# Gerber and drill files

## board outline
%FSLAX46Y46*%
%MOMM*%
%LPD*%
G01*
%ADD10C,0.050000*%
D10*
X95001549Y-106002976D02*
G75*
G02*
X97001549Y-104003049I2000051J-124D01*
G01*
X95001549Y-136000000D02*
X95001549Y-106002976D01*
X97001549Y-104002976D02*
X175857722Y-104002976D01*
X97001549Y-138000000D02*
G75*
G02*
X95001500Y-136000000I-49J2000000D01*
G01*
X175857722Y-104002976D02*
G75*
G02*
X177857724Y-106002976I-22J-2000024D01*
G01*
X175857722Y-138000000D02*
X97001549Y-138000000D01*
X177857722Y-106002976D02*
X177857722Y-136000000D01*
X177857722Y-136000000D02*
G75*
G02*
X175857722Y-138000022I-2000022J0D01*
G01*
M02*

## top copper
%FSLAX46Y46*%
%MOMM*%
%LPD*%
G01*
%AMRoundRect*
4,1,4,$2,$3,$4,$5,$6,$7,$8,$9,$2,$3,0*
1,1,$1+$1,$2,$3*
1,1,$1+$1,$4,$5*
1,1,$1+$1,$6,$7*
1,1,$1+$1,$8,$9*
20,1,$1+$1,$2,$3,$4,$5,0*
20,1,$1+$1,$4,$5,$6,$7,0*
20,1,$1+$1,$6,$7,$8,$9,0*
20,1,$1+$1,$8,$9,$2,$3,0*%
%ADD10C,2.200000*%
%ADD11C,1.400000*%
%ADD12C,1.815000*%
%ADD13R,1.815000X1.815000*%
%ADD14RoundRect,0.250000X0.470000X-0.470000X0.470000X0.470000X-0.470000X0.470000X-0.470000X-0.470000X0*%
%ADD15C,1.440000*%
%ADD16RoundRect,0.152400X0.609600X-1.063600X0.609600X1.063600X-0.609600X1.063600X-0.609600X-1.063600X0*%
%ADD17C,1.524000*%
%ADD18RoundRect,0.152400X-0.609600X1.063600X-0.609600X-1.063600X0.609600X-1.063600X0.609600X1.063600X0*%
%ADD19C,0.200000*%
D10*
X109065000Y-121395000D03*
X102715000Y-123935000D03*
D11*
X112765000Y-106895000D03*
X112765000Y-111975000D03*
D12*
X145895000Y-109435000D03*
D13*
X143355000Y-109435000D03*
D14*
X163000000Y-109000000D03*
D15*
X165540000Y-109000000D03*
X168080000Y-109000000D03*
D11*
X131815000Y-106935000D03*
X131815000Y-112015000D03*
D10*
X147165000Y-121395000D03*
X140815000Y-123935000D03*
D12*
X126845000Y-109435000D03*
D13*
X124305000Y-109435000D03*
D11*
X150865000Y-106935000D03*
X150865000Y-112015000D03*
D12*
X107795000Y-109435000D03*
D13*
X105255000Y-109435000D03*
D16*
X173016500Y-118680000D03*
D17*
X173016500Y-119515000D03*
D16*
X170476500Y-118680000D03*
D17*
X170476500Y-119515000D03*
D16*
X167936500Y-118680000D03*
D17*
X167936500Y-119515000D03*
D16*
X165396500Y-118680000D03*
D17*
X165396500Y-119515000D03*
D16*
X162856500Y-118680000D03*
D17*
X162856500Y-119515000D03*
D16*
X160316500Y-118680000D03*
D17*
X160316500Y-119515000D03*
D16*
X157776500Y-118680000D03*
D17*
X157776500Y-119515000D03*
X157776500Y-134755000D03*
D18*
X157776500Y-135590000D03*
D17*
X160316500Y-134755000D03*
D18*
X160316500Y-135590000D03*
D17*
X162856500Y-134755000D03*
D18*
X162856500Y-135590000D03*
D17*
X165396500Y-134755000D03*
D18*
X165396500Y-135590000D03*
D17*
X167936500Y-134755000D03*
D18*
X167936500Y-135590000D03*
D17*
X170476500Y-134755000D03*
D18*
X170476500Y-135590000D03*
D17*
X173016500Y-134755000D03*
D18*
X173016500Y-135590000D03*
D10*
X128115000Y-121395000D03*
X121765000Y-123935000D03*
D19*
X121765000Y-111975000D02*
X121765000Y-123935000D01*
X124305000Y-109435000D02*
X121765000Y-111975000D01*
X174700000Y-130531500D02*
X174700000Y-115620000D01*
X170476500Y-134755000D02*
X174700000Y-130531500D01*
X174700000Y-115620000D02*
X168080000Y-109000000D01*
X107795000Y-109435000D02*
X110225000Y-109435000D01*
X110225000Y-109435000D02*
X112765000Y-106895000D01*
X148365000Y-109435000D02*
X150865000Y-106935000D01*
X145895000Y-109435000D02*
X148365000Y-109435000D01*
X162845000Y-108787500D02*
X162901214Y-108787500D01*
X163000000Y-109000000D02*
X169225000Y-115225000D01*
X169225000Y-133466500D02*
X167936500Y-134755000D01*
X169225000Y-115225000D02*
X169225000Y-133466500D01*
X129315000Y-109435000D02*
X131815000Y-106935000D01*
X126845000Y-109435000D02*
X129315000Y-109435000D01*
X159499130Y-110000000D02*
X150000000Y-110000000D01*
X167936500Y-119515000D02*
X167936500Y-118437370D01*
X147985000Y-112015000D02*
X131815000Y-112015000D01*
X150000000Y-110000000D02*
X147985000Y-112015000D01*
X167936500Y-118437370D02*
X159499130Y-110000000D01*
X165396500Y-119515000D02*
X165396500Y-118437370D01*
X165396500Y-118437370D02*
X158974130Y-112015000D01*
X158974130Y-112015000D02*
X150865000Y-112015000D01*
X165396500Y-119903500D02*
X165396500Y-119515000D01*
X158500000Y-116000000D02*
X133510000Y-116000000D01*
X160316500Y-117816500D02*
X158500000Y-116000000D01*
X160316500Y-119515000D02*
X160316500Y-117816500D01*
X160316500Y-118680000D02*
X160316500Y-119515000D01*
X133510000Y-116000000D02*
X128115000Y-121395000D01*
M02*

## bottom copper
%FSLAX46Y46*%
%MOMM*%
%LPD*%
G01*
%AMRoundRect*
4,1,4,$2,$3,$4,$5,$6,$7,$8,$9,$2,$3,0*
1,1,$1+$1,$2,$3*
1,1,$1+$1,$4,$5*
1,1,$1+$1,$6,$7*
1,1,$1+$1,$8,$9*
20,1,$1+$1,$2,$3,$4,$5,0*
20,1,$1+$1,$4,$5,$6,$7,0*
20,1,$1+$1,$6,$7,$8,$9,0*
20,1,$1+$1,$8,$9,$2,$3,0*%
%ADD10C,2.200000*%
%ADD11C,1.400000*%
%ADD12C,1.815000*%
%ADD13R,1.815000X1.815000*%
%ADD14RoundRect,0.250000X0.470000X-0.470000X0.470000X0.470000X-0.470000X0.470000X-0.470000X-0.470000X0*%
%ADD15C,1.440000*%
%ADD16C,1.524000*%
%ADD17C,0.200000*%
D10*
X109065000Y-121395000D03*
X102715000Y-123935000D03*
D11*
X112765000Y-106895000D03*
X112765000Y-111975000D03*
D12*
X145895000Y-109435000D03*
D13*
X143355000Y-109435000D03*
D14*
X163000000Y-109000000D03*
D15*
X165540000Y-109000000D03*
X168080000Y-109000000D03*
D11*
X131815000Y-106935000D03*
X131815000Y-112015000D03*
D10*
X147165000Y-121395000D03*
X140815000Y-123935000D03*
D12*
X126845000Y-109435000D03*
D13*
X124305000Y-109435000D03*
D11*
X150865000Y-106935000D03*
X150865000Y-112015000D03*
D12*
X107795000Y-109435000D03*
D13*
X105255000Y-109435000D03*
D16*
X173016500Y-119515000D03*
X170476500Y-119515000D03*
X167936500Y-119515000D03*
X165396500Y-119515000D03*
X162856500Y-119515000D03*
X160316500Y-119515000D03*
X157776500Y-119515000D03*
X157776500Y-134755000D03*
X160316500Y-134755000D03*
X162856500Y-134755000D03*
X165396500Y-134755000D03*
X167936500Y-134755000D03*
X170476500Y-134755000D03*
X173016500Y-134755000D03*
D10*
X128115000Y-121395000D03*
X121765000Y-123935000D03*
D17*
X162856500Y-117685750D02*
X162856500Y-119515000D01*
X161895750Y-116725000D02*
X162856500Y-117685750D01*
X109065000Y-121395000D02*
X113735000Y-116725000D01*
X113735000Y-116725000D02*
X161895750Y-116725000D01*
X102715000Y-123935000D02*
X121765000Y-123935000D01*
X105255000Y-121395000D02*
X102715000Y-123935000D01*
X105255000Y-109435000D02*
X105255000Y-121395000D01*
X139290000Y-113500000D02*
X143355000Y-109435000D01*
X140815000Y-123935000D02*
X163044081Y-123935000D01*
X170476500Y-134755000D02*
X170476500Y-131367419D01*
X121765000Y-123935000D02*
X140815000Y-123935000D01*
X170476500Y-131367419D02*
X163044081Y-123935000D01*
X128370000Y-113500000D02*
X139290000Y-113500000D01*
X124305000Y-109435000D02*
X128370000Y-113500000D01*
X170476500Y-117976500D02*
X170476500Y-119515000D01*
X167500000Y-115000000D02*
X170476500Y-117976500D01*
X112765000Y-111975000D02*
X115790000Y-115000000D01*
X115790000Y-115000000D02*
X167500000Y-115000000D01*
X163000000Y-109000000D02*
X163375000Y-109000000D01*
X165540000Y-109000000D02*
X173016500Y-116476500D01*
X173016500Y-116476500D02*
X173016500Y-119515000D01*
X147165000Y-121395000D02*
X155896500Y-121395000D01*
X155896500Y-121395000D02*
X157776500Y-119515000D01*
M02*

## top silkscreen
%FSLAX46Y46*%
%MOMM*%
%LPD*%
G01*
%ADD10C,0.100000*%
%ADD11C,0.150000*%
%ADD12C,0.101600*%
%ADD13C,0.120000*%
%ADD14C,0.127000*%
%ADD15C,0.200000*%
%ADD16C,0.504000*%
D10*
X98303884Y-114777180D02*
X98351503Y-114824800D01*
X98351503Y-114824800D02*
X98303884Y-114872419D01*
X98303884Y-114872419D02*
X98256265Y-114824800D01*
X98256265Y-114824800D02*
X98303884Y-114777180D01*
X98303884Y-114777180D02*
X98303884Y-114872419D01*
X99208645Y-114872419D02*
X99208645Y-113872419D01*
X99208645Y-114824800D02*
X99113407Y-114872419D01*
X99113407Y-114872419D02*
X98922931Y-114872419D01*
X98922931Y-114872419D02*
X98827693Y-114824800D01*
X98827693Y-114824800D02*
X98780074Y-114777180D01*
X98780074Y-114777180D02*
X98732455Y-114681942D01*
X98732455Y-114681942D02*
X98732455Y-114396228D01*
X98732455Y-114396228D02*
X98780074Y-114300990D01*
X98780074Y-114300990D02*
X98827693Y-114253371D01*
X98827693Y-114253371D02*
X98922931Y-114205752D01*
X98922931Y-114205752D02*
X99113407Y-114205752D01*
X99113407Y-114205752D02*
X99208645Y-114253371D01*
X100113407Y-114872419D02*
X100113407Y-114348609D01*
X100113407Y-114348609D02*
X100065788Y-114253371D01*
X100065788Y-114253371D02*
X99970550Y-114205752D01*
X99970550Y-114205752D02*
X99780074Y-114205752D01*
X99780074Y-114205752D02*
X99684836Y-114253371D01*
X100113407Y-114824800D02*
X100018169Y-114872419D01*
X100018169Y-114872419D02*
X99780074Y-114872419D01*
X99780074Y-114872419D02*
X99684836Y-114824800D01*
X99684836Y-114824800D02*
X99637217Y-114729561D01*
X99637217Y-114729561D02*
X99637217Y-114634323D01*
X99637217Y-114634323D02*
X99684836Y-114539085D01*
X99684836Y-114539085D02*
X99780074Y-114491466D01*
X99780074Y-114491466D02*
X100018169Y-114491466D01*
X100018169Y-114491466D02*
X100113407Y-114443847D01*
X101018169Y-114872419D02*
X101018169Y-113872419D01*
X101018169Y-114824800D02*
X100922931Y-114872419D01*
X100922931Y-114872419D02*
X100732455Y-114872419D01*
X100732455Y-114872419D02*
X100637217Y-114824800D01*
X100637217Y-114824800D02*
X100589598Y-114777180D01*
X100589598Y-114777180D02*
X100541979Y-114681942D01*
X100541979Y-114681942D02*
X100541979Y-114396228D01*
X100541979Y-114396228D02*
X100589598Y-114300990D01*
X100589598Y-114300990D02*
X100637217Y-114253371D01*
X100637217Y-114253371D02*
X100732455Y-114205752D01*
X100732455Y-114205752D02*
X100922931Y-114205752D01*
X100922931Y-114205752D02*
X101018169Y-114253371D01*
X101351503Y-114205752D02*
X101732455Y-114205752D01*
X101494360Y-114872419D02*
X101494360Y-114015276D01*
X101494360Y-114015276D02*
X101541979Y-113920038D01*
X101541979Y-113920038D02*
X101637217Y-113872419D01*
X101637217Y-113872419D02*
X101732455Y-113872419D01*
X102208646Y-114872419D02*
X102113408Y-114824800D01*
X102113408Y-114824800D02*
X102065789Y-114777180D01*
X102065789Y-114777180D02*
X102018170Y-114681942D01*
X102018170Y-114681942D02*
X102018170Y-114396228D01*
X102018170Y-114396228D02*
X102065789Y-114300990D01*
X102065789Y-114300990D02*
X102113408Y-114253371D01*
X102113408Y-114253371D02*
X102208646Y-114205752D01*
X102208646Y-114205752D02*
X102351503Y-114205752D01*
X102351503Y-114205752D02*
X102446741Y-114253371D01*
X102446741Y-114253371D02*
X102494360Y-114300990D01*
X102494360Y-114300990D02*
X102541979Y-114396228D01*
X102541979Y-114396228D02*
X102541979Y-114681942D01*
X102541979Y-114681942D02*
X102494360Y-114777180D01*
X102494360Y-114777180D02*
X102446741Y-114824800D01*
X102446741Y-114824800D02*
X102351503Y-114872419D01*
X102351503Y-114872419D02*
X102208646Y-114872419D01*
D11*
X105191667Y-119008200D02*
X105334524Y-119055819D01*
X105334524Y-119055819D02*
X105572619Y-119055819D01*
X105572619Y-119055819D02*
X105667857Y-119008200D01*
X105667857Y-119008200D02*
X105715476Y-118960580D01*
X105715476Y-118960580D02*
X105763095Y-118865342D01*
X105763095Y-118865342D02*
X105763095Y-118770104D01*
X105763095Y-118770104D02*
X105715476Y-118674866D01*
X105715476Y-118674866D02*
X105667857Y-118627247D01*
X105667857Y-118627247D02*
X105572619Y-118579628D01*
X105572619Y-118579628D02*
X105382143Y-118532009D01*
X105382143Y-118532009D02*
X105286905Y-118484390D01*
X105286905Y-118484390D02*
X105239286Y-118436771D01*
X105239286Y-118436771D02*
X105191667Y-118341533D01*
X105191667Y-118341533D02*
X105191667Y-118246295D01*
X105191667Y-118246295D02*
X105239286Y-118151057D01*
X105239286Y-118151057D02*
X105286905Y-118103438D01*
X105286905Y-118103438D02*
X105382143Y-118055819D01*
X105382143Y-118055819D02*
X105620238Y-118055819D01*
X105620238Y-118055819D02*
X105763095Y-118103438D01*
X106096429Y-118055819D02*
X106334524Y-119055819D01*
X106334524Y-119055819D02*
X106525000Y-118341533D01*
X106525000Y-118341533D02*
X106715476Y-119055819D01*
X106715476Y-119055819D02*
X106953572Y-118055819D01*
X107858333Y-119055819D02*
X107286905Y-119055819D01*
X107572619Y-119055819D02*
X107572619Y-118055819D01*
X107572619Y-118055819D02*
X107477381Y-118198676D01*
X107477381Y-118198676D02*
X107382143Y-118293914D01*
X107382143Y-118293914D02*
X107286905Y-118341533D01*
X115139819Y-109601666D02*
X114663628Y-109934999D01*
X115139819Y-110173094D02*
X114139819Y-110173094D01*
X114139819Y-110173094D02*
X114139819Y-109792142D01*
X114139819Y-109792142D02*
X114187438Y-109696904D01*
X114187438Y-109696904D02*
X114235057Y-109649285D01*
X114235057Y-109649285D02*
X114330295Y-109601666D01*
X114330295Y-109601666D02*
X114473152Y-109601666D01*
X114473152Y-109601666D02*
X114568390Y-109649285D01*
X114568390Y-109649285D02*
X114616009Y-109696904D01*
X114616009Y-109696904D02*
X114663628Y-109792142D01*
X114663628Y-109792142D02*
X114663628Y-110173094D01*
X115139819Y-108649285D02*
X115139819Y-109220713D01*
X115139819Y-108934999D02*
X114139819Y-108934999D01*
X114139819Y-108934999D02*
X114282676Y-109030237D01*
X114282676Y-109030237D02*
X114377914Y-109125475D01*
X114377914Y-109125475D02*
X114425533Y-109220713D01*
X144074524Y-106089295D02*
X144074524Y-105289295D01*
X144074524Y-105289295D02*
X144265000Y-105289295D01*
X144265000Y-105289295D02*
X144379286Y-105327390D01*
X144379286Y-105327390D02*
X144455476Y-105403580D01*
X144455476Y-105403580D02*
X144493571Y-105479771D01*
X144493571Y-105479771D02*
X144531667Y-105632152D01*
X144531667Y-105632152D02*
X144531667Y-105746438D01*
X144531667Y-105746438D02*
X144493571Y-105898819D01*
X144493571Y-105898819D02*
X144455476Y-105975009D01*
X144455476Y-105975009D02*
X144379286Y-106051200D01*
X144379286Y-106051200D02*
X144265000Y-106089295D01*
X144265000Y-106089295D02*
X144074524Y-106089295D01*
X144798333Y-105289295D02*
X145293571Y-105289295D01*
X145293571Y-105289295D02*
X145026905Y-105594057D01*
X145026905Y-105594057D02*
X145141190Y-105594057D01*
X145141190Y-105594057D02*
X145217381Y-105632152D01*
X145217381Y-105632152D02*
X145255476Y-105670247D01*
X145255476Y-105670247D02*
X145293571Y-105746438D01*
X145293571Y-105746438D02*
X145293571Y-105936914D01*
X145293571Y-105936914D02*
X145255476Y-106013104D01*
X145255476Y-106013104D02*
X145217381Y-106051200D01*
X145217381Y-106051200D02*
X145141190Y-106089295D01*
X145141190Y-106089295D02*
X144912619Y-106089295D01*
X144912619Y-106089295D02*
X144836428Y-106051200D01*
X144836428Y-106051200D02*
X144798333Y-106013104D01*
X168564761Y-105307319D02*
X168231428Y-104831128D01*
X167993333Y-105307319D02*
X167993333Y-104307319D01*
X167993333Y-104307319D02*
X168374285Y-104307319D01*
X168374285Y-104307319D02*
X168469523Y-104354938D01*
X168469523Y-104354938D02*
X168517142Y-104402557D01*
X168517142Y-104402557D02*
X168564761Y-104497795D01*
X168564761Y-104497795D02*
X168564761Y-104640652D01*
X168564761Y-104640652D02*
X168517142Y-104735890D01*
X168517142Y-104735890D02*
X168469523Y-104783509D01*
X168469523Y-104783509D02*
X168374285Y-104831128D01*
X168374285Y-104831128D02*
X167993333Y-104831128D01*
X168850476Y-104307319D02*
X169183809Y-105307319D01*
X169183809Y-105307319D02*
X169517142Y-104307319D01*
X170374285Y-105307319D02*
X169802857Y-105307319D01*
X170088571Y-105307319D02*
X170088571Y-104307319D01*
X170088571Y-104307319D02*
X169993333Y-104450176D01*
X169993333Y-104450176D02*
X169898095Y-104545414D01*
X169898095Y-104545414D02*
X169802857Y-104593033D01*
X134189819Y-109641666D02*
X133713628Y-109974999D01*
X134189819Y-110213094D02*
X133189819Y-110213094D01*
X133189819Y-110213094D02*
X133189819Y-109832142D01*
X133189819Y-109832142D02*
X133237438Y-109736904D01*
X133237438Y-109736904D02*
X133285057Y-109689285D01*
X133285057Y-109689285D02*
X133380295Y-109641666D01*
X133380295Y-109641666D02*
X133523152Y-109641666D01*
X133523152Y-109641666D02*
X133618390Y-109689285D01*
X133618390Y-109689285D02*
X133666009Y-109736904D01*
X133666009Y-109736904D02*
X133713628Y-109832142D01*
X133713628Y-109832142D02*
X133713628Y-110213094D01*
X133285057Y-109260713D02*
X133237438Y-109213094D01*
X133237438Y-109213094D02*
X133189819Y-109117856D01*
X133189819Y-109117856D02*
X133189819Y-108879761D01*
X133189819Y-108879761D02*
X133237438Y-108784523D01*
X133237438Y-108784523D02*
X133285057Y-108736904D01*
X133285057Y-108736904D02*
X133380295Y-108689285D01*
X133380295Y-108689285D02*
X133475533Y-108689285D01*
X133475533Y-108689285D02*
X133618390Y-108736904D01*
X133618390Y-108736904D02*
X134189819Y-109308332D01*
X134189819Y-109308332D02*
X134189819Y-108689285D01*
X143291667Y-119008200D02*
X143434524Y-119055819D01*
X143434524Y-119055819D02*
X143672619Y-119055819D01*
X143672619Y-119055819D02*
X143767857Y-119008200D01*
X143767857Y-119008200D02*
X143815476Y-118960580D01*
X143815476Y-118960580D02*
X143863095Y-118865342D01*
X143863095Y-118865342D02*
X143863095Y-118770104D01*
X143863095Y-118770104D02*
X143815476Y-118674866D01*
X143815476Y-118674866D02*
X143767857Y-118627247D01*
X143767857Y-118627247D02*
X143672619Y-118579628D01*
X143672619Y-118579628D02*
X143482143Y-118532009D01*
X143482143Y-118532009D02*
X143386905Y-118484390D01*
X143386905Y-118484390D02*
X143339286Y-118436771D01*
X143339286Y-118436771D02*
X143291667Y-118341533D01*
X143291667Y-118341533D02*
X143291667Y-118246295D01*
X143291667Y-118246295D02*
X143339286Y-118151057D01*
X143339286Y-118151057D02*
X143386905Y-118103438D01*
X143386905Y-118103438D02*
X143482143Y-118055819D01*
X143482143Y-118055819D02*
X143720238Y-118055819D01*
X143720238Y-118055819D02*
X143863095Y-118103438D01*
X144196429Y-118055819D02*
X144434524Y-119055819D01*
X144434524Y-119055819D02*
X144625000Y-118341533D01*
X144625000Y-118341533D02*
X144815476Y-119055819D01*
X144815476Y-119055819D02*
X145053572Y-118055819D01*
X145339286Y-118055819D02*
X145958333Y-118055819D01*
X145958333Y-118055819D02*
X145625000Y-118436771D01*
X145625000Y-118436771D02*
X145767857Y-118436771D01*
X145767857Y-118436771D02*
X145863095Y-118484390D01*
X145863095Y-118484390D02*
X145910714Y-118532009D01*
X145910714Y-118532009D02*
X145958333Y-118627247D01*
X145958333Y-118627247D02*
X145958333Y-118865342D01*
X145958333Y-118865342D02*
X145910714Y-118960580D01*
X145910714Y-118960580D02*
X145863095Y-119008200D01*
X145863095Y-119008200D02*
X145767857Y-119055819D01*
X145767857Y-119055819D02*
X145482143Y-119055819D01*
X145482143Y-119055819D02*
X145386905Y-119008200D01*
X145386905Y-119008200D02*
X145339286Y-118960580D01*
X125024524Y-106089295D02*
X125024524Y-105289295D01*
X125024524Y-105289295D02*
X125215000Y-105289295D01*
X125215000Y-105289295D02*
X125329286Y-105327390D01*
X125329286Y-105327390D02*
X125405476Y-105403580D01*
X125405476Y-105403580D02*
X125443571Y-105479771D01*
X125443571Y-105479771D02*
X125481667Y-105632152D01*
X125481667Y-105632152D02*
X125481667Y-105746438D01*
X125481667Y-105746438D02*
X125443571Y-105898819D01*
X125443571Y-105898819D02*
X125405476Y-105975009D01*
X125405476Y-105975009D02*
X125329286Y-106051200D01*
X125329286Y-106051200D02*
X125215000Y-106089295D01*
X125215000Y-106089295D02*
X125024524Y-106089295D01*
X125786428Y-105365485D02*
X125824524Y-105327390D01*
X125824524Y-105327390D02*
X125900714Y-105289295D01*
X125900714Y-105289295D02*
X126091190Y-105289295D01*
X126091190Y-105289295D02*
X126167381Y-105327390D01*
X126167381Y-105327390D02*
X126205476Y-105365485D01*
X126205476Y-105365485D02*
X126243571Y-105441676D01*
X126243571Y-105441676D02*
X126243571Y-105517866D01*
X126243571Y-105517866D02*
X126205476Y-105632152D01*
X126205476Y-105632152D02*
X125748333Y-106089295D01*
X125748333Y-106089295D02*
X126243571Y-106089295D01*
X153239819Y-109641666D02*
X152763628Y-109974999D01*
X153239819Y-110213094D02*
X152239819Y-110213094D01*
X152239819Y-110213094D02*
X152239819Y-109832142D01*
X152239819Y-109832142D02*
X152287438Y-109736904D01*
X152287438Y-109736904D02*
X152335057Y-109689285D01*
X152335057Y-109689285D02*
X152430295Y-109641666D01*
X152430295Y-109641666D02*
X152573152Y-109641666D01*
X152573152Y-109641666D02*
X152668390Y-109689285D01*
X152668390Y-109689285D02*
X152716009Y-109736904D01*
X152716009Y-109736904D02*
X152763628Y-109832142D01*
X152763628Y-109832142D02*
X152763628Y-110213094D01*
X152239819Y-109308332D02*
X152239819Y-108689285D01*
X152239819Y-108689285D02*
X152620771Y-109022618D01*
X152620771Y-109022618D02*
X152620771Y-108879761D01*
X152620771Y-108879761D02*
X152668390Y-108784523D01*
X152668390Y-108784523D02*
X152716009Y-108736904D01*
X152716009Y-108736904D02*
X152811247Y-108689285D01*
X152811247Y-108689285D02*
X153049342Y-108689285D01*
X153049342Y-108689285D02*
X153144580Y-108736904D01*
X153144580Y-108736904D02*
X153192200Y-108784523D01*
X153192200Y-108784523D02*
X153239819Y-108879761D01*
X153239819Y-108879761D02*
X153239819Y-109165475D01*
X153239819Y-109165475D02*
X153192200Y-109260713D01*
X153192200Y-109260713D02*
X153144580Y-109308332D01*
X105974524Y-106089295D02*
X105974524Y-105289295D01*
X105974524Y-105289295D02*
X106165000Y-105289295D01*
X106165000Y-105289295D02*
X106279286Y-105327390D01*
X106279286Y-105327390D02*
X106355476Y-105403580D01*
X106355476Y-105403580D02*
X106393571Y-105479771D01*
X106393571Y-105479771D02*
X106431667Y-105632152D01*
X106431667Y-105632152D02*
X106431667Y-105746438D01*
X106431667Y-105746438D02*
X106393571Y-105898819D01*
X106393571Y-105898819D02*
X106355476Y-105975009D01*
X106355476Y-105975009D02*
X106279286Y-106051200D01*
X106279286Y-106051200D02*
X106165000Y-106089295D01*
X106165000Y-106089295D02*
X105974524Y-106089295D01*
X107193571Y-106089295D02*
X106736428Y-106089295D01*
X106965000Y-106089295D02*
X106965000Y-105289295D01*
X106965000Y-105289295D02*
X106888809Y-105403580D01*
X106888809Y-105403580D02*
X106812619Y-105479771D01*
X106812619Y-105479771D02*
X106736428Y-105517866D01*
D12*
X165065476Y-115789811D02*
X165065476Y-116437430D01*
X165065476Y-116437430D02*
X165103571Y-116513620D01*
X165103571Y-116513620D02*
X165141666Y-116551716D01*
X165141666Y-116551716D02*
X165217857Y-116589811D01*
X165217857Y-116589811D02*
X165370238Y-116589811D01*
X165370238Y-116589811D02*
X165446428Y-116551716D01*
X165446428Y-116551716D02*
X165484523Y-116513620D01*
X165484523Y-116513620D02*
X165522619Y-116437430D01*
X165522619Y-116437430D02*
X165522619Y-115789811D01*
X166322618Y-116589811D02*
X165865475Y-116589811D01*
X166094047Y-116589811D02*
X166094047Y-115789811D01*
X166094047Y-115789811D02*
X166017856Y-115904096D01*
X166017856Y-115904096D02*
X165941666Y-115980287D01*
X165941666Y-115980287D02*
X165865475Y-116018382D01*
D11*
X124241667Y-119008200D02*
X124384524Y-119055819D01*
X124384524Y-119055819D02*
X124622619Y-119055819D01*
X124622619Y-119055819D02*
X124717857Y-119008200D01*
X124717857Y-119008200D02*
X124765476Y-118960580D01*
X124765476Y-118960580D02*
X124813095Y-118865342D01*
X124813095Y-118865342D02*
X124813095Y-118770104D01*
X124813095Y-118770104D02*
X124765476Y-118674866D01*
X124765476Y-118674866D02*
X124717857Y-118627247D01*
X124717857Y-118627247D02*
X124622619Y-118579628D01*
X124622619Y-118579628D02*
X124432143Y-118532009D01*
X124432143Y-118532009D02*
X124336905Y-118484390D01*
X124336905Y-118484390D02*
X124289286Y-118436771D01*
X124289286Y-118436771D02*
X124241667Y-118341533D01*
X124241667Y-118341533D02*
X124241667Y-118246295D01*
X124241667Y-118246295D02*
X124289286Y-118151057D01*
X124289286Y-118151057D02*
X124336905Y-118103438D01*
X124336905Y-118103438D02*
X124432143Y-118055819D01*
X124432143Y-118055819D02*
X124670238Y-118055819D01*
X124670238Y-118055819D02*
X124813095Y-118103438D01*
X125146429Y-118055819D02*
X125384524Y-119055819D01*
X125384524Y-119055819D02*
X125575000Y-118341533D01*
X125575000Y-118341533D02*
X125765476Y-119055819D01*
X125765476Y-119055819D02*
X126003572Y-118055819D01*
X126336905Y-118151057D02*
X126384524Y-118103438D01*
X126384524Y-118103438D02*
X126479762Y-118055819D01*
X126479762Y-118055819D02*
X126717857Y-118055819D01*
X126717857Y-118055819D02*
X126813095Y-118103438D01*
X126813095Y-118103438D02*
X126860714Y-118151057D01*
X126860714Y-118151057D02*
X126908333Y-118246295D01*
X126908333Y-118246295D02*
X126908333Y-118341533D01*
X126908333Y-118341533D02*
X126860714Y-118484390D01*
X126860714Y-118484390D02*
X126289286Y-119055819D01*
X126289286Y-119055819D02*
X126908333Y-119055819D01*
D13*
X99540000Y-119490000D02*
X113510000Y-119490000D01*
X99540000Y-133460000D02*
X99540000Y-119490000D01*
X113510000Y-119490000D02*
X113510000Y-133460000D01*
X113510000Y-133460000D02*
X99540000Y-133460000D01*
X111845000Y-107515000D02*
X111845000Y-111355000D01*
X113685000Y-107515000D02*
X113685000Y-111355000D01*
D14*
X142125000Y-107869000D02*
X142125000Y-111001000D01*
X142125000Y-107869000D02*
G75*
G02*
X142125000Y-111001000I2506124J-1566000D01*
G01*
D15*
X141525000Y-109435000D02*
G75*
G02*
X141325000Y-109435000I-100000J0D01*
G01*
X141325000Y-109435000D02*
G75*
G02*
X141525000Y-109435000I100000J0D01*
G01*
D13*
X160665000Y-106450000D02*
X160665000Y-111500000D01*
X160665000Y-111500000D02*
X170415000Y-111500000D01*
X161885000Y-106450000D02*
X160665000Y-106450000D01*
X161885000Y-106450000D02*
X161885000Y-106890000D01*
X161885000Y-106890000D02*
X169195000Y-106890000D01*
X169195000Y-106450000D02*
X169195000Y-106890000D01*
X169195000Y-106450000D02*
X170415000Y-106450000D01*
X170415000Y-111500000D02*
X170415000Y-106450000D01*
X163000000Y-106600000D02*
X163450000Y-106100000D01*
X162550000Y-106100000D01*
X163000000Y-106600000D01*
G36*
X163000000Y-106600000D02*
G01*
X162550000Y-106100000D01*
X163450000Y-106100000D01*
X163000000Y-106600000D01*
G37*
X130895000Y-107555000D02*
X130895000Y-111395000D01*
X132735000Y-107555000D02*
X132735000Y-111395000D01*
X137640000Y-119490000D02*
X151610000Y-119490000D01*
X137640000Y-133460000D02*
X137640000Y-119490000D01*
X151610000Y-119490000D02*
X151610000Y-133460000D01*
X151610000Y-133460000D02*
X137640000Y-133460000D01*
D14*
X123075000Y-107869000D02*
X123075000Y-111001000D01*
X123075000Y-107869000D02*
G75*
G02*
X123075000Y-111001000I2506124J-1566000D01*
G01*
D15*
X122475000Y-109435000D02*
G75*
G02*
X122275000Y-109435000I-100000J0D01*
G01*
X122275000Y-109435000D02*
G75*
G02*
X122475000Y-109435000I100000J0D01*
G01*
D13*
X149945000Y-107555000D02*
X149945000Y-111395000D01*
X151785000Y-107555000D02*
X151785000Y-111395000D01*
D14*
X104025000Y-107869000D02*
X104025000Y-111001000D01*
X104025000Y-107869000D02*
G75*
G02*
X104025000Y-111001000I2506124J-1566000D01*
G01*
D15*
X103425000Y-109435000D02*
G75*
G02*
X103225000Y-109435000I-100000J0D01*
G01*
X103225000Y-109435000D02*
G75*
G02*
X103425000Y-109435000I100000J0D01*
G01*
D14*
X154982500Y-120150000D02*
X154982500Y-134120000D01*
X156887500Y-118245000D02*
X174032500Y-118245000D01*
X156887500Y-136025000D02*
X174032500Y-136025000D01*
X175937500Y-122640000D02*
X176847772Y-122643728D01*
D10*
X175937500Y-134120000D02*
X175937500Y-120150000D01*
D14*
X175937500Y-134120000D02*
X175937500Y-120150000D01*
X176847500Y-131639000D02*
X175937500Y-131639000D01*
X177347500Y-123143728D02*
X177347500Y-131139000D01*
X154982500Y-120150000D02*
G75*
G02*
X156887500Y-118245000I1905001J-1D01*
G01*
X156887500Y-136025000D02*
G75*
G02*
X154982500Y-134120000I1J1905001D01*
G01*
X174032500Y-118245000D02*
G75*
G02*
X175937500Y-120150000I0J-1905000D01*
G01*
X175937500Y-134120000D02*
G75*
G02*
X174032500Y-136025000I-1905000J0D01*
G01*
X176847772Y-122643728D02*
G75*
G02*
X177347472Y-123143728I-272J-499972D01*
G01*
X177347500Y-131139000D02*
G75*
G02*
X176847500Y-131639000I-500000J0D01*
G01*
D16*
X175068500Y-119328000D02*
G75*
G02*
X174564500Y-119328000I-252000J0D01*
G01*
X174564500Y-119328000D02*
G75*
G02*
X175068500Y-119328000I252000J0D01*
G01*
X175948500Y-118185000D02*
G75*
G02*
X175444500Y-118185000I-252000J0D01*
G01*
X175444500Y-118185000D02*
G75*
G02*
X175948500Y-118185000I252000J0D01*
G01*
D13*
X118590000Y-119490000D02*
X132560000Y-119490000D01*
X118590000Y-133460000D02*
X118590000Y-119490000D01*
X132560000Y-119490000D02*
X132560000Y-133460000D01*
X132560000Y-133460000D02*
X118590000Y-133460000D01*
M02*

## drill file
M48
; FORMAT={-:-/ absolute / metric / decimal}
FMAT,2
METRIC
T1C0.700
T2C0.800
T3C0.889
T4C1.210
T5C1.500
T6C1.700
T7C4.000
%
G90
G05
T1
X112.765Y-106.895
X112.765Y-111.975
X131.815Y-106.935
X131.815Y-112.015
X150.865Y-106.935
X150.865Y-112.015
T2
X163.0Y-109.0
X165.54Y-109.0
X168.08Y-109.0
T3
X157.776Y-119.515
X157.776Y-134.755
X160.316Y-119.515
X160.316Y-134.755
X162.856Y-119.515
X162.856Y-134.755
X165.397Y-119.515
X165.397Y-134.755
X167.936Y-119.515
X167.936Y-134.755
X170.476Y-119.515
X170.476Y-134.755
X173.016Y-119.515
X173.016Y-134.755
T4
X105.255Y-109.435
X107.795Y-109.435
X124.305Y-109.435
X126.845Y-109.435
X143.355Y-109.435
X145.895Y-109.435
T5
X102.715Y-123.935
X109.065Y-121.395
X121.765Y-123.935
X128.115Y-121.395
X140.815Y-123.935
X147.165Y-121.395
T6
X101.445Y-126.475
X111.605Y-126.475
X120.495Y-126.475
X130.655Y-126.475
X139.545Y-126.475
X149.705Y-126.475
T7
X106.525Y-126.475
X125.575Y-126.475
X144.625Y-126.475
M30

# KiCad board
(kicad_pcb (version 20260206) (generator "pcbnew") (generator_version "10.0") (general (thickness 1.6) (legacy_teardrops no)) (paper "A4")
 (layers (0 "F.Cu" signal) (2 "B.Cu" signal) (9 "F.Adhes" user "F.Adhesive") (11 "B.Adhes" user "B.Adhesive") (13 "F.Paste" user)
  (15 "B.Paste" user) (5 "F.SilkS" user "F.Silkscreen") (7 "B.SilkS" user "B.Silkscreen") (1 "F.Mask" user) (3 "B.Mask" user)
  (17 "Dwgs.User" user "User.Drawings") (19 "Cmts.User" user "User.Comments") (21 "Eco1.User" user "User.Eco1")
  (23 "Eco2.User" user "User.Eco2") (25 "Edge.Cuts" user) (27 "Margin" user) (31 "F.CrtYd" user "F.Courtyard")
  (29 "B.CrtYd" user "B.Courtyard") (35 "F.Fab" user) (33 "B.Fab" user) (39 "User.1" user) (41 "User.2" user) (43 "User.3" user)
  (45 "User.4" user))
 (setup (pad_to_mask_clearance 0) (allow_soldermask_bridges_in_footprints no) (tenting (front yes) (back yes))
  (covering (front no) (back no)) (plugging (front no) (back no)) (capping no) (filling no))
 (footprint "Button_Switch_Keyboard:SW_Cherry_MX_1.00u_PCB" (layer "F.Cu") (at 109.065 121.395)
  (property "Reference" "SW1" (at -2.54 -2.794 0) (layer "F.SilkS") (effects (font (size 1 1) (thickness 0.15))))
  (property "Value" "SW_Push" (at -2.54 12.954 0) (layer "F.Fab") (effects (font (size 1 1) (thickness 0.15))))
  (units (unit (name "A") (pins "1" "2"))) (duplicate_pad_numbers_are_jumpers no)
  (fp_line (start -9.525 -1.905) (end 4.445 -1.905) (stroke (width 0.12) (type solid)) (layer "F.SilkS"))
  (fp_line (start -9.525 12.065) (end -9.525 -1.905) (stroke (width 0.12) (type solid)) (layer "F.SilkS"))
  (fp_line (start 4.445 -1.905) (end 4.445 12.065) (stroke (width 0.12) (type solid)) (layer "F.SilkS"))
  (fp_line (start 4.445 12.065) (end -9.525 12.065) (stroke (width 0.12) (type solid)) (layer "F.SilkS"))
  (pad "" np_thru_hole circle (at -7.62 5.08) (size 1.7 1.7) (drill 1.7) (layers "*.Cu" "*.Mask"))
  (pad "" np_thru_hole circle (at -2.54 5.08) (size 4 4) (drill 4) (layers "*.Cu" "*.Mask"))
  (pad "" np_thru_hole circle (at 2.54 5.08) (size 1.7 1.7) (drill 1.7) (layers "*.Cu" "*.Mask"))
  (pad "1" thru_hole circle (at 0 0) (size 2.2 2.2) (drill 1.5) (layers "*.Cu" "*.Mask") (remove_unused_layers no) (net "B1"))
  (pad "2" thru_hole circle (at -6.35 2.54) (size 2.2 2.2) (drill 1.5) (layers "*.Cu" "*.Mask") (remove_unused_layers no) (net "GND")))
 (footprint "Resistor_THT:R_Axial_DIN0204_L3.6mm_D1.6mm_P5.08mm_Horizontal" (layer "F.Cu") (at 112.765 106.895 -90)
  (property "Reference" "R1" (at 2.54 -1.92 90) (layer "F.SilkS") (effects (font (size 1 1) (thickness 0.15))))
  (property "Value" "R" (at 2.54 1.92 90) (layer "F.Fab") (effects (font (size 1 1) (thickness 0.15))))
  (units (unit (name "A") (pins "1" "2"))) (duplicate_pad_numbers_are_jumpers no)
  (fp_line (start 0.62 0.92) (end 4.46 0.92) (stroke (width 0.12) (type solid)) (layer "F.SilkS"))
  (fp_line (start 0.62 -0.92) (end 4.46 -0.92) (stroke (width 0.12) (type solid)) (layer "F.SilkS"))
  (pad "1" thru_hole circle (at 0 0 270) (size 1.4 1.4) (drill 0.7) (layers "*.Cu" "*.Mask") (remove_unused_layers no) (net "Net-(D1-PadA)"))
  (pad "2" thru_hole circle (at 5.08 0 270) (size 1.4 1.4) (drill 0.7) (layers "*.Cu" "*.Mask") (remove_unused_layers no) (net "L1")))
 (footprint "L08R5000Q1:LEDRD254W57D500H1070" (layer "F.Cu") (at 144.625 109.435)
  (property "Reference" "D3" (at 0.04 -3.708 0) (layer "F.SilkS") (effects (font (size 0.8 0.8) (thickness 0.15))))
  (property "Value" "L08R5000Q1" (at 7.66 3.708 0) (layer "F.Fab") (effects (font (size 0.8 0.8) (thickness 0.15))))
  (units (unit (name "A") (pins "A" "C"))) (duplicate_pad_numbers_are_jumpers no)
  (fp_line (start -2.5 -1.566) (end -2.5 1.566) (stroke (width 0.127) (type solid)) (layer "F.SilkS"))
  (fp_arc (start -2.5 -1.566) (mid 2.961291 0) (end -2.5 1.566) (stroke (width 0.127) (type solid)) (layer "F.SilkS"))
  (fp_circle (center -3.2 0) (end -3.1 0) (stroke (width 0.2) (type solid)) (fill no) (layer "F.SilkS"))
  (pad "A" thru_hole circle (at 1.27 0) (size 1.815 1.815) (drill 1.21) (layers "*.Cu" "*.Mask") (remove_unused_layers no)
   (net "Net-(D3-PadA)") (solder_mask_margin 0.102))
  (pad "C" thru_hole rect (at -1.27 0) (size 1.815 1.815) (drill 1.21) (layers "*.Cu" "*.Mask") (remove_unused_layers no) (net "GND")
   (solder_mask_margin 0.102)))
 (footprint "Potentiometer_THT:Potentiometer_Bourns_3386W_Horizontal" (layer "F.Cu") (at 163 109)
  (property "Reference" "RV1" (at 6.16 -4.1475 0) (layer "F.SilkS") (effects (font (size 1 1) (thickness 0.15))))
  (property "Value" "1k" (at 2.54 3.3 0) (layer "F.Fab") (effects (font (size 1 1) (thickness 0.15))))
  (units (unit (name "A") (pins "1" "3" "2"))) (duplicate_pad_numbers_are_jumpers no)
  (fp_line (start -2.335 -2.55) (end -2.335 2.5) (stroke (width 0.12) (type default)) (layer "F.SilkS"))
  (fp_line (start -2.335 2.5) (end 7.415 2.5) (stroke (width 0.12) (type default)) (layer "F.SilkS"))
  (fp_line (start -1.115 -2.55) (end -2.335 -2.55) (stroke (width 0.12) (type default)) (layer "F.SilkS"))
  (fp_line (start -1.115 -2.55) (end -1.115 -2.11) (stroke (width 0.12) (type default)) (layer "F.SilkS"))
  (fp_line (start -1.115 -2.11) (end 6.195 -2.11) (stroke (width 0.12) (type default)) (layer "F.SilkS"))
  (fp_line (start 6.195 -2.55) (end 6.195 -2.11) (stroke (width 0.12) (type default)) (layer "F.SilkS"))
  (fp_line (start 6.195 -2.55) (end 7.415 -2.55) (stroke (width 0.12) (type default)) (layer "F.SilkS"))
  (fp_line (start 7.415 2.5) (end 7.415 -2.55) (stroke (width 0.12) (type default)) (layer "F.SilkS"))
  (fp_poly (pts (xy 0 -2.4) (xy 0.45 -2.9) (xy -0.45 -2.9)) (stroke (width 0.12) (type solid)) (fill yes) (layer "F.SilkS"))
  (pad "1" thru_hole roundrect (at 0 0 90) (size 1.44 1.44) (drill 0.8) (layers "*.Cu" "*.Mask") (remove_unused_layers no)
   (roundrect_rratio 0.1736111111) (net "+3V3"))
  (pad "2" thru_hole circle (at 2.54 0 90) (size 1.44 1.44) (drill 0.8) (layers "*.Cu" "*.Mask") (remove_unused_layers no) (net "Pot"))
  (pad "3" thru_hole circle (at 5.08 0 90) (size 1.44 1.44) (drill 0.8) (layers "*.Cu" "*.Mask") (remove_unused_layers no) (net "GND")))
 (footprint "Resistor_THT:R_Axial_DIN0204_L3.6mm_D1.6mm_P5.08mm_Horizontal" (layer "F.Cu") (at 131.815 106.935 -90)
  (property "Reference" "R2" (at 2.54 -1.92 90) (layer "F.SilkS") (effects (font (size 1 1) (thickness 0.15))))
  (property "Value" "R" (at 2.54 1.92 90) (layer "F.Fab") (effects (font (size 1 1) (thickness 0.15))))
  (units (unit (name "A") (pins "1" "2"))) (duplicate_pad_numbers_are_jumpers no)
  (fp_line (start 0.62 0.92) (end 4.46 0.92) (stroke (width 0.12) (type solid)) (layer "F.SilkS"))
  (fp_line (start 0.62 -0.92) (end 4.46 -0.92) (stroke (width 0.12) (type solid)) (layer "F.SilkS"))
  (pad "1" thru_hole circle (at 0 0 270) (size 1.4 1.4) (drill 0.7) (layers "*.Cu" "*.Mask") (remove_unused_layers no) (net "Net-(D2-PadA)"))
  (pad "2" thru_hole circle (at 5.08 0 270) (size 1.4 1.4) (drill 0.7) (layers "*.Cu" "*.Mask") (remove_unused_layers no) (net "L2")))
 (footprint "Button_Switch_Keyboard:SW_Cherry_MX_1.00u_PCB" (layer "F.Cu") (at 147.165 121.395)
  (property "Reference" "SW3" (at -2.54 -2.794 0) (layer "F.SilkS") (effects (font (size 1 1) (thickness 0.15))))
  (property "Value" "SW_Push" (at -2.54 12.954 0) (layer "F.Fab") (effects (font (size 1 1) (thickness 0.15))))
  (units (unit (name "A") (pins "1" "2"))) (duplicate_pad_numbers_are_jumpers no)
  (fp_line (start -9.525 -1.905) (end 4.445 -1.905) (stroke (width 0.12) (type solid)) (layer "F.SilkS"))
  (fp_line (start -9.525 12.065) (end -9.525 -1.905) (stroke (width 0.12) (type solid)) (layer "F.SilkS"))
  (fp_line (start 4.445 -1.905) (end 4.445 12.065) (stroke (width 0.12) (type solid)) (layer "F.SilkS"))
  (fp_line (start 4.445 12.065) (end -9.525 12.065) (stroke (width 0.12) (type solid)) (layer "F.SilkS"))
  (pad "" np_thru_hole circle (at -7.62 5.08) (size 1.7 1.7) (drill 1.7) (layers "*.Cu" "*.Mask"))
  (pad "" np_thru_hole circle (at -2.54 5.08) (size 4 4) (drill 4) (layers "*.Cu" "*.Mask"))
  (pad "" np_thru_hole circle (at 2.54 5.08) (size 1.7 1.7) (drill 1.7) (layers "*.Cu" "*.Mask"))
  (pad "1" thru_hole circle (at 0 0) (size 2.2 2.2) (drill 1.5) (layers "*.Cu" "*.Mask") (remove_unused_layers no) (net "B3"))
  (pad "2" thru_hole circle (at -6.35 2.54) (size 2.2 2.2) (drill 1.5) (layers "*.Cu" "*.Mask") (remove_unused_layers no) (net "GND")))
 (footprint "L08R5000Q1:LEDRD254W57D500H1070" (layer "F.Cu") (at 125.575 109.435)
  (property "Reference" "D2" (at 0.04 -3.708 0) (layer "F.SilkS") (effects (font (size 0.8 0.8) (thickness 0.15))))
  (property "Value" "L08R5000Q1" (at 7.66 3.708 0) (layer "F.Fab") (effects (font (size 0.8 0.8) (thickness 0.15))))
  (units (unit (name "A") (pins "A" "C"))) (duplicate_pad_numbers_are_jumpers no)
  (fp_line (start -2.5 -1.566) (end -2.5 1.566) (stroke (width 0.127) (type solid)) (layer "F.SilkS"))
  (fp_arc (start -2.5 -1.566) (mid 2.961291 0) (end -2.5 1.566) (stroke (width 0.127) (type solid)) (layer "F.SilkS"))
  (fp_circle (center -3.2 0) (end -3.1 0) (stroke (width 0.2) (type solid)) (fill no) (layer "F.SilkS"))
  (pad "A" thru_hole circle (at 1.27 0) (size 1.815 1.815) (drill 1.21) (layers "*.Cu" "*.Mask") (remove_unused_layers no)
   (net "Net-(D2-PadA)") (solder_mask_margin 0.102))
  (pad "C" thru_hole rect (at -1.27 0) (size 1.815 1.815) (drill 1.21) (layers "*.Cu" "*.Mask") (remove_unused_layers no) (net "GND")
   (solder_mask_margin 0.102)))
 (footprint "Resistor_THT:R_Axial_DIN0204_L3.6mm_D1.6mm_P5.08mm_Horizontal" (layer "F.Cu") (at 150.865 106.935 -90)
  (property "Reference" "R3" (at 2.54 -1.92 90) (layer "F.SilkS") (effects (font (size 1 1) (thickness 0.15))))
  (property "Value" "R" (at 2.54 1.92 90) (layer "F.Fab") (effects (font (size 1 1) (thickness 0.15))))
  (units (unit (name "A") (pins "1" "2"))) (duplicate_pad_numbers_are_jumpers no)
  (fp_line (start 0.62 0.92) (end 4.46 0.92) (stroke (width 0.12) (type solid)) (layer "F.SilkS"))
  (fp_line (start 0.62 -0.92) (end 4.46 -0.92) (stroke (width 0.12) (type solid)) (layer "F.SilkS"))
  (pad "1" thru_hole circle (at 0 0 270) (size 1.4 1.4) (drill 0.7) (layers "*.Cu" "*.Mask") (remove_unused_layers no) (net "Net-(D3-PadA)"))
  (pad "2" thru_hole circle (at 5.08 0 270) (size 1.4 1.4) (drill 0.7) (layers "*.Cu" "*.Mask") (remove_unused_layers no) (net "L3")))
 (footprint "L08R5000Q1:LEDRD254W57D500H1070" (layer "F.Cu") (at 106.525 109.435)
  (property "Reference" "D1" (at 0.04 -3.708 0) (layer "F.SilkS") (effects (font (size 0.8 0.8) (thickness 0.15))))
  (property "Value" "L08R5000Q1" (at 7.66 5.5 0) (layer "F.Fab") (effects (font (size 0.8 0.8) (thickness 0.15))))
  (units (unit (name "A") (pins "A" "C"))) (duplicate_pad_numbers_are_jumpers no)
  (fp_line (start -2.5 -1.566) (end -2.5 1.566) (stroke (width 0.127) (type solid)) (layer "F.SilkS"))
  (fp_arc (start -2.5 -1.566) (mid 2.961291 0) (end -2.5 1.566) (stroke (width 0.127) (type solid)) (layer "F.SilkS"))
  (fp_circle (center -3.2 0) (end -3.1 0) (stroke (width 0.2) (type solid)) (fill no) (layer "F.SilkS"))
  (pad "A" thru_hole circle (at 1.27 0) (size 1.815 1.815) (drill 1.21) (layers "*.Cu" "*.Mask") (remove_unused_layers no)
   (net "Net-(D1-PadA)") (solder_mask_margin 0.102))
  (pad "C" thru_hole rect (at -1.27 0) (size 1.815 1.815) (drill 1.21) (layers "*.Cu" "*.Mask") (remove_unused_layers no) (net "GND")
   (solder_mask_margin 0.102)))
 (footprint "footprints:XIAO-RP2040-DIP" (layer "F.Cu") (at 165.3965 127.135)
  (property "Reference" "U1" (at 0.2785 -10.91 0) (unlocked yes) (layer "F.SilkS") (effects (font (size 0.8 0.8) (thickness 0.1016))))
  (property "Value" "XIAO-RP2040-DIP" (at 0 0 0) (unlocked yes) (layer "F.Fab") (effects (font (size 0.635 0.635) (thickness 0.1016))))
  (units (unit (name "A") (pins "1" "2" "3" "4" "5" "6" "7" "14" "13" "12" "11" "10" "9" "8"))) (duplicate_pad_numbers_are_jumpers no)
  (fp_line (start -10.414 -6.985) (end -10.414 6.985) (stroke (width 0.127) (type solid)) (layer "F.SilkS"))
  (fp_line (start -8.509 -8.89) (end 8.636 -8.89) (stroke (width 0.127) (type solid)) (layer "F.SilkS"))
  (fp_line (start -8.509 8.89) (end 8.636 8.89) (stroke (width 0.127) (type solid)) (layer "F.SilkS"))
  (fp_line (start 10.541 -4.495) (end 11.451272 -4.491272) (stroke (width 0.127) (type solid)) (layer "F.SilkS"))
  (fp_line (start 10.541 6.985) (end 10.541 -6.985) (stroke (width 0.1) (type solid)) (layer "F.SilkS"))
  (fp_line (start 10.541 6.985) (end 10.541 -6.985) (stroke (width 0.127) (type solid)) (layer "F.SilkS"))
  (fp_line (start 11.451 4.504) (end 10.541 4.504) (stroke (width 0.127) (type solid)) (layer "F.SilkS"))
  (fp_line (start 11.951 -3.991272) (end 11.951 4.004) (stroke (width 0.127) (type solid)) (layer "F.SilkS"))
  (fp_arc (start -10.414 -6.985) (mid -9.856038 -8.332038) (end -8.509 -8.89) (stroke (width 0.127) (type solid)) (layer "F.SilkS"))
  (fp_arc (start -8.509 8.89) (mid -9.856038 8.332038) (end -10.414 6.985) (stroke (width 0.127) (type solid)) (layer "F.SilkS"))
  (fp_arc (start 8.636 -8.89) (mid 9.983038 -8.332038) (end 10.541 -6.985) (stroke (width 0.127) (type solid)) (layer "F.SilkS"))
  (fp_arc (start 10.541 6.985) (mid 9.983038 8.332038) (end 8.636 8.89) (stroke (width 0.127) (type solid)) (layer "F.SilkS"))
  (fp_arc (start 11.451272 -4.491272) (mid 11.804644 -4.344724) (end 11.951 -3.991272) (stroke (width 0.127) (type default))
   (layer "F.SilkS"))
  (fp_arc (start 11.951 4.004) (mid 11.804553 4.357553) (end 11.451 4.504) (stroke (width 0.127) (type default)) (layer "F.SilkS"))
  (fp_circle (center 9.42 -7.807) (end 9.674 -7.807) (stroke (width 0.5) (type solid)) (fill yes) (layer "F.SilkS"))
  (fp_circle (center 10.3 -8.95) (end 10.554 -8.95) (stroke (width 0.5) (type solid)) (fill yes) (layer "F.SilkS"))
  (pad "1" smd roundrect (at 7.62 -8.455 90) (size 2.432 1.524) (layers "F.Cu" "F.Mask") (roundrect_rratio 0.1) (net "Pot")
   (thermal_bridge_angle 45))
  (pad "1" thru_hole circle (at 7.62 -7.62 90) (size 1.524 1.524) (drill 0.889) (layers "*.Cu" "*.Mask") (remove_unused_layers no)
   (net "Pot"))
  (pad "2" smd roundrect (at 5.08 -8.455 90) (size 2.432 1.524) (layers "F.Cu" "F.Mask") (roundrect_rratio 0.1) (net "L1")
   (thermal_bridge_angle 45))
  (pad "2" thru_hole circle (at 5.08 -7.62 90) (size 1.524 1.524) (drill 0.889) (layers "*.Cu" "*.Mask") (remove_unused_layers no)
   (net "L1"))
  (pad "3" smd roundrect (at 2.54 -8.455 90) (size 2.432 1.524) (layers "F.Cu" "F.Mask") (roundrect_rratio 0.1) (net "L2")
   (thermal_bridge_angle 45))
  (pad "3" thru_hole circle (at 2.54 -7.62 90) (size 1.524 1.524) (drill 0.889) (layers "*.Cu" "*.Mask") (remove_unused_layers no)
   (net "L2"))
  (pad "4" smd roundrect (at 0 -8.455 90) (size 2.432 1.524) (layers "F.Cu" "F.Mask") (roundrect_rratio 0.1) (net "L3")
   (thermal_bridge_angle 45))
  (pad "4" thru_hole circle (at 0 -7.62 90) (size 1.524 1.524) (drill 0.889) (layers "*.Cu" "*.Mask") (remove_unused_layers no) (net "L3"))
  (pad "5" smd roundrect (at -2.54 -8.455 90) (size 2.432 1.524) (layers "F.Cu" "F.Mask") (roundrect_rratio 0.1) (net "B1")
   (thermal_bridge_angle 45))
  (pad "5" thru_hole circle (at -2.54 -7.62 90) (size 1.524 1.524) (drill 0.889) (layers "*.Cu" "*.Mask") (remove_unused_layers no)
   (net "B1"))
  (pad "6" smd roundrect (at -5.08 -8.455 90) (size 2.432 1.524) (layers "F.Cu" "F.Mask") (roundrect_rratio 0.1) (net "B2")
   (thermal_bridge_angle 45))
  (pad "6" thru_hole circle (at -5.08 -7.62 90) (size 1.524 1.524) (drill 0.889) (layers "*.Cu" "*.Mask") (remove_unused_layers no)
   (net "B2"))
  (pad "7" smd roundrect (at -7.62 -8.455 90) (size 2.432 1.524) (layers "F.Cu" "F.Mask") (roundrect_rratio 0.1) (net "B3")
   (thermal_bridge_angle 45))
  (pad "7" thru_hole circle (at -7.62 -7.62 90) (size 1.524 1.524) (drill 0.889) (layers "*.Cu" "*.Mask") (remove_unused_layers no)
   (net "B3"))
  (pad "8" thru_hole circle (at -7.62 7.62 270) (size 1.524 1.524) (drill 0.889) (layers "*.Cu" "*.Mask") (remove_unused_layers no)
   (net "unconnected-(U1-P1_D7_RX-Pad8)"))
  (pad "8" smd roundrect (at -7.62 8.455 270) (size 2.432 1.524) (layers "F.Cu" "F.Mask") (roundrect_rratio 0.1)
   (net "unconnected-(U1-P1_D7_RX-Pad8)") (thermal_bridge_angle 45))
  (pad "9" thru_hole circle (at -5.08 7.62 270) (size 1.524 1.524) (drill 0.889) (layers "*.Cu" "*.Mask") (remove_unused_layers no)
   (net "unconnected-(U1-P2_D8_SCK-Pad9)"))
  (pad "9" smd roundrect (at -5.08 8.455 270) (size 2.432 1.524) (layers "F.Cu" "F.Mask") (roundrect_rratio 0.1)
   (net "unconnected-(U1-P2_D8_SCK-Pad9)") (thermal_bridge_angle 45))
  (pad "10" thru_hole circle (at -2.54 7.62 270) (size 1.524 1.524) (drill 0.889) (layers "*.Cu" "*.Mask") (remove_unused_layers no)
   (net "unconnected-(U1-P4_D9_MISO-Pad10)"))
  (pad "10" smd roundrect (at -2.54 8.455 270) (size 2.432 1.524) (layers "F.Cu" "F.Mask") (roundrect_rratio 0.1)
   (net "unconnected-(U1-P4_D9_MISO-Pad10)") (thermal_bridge_angle 45))
  (pad "11" thru_hole circle (at 0 7.62 270) (size 1.524 1.524) (drill 0.889) (layers "*.Cu" "*.Mask") (remove_unused_layers no)
   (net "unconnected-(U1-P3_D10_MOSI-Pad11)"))
  (pad "11" smd roundrect (at 0 8.455 270) (size 2.432 1.524) (layers "F.Cu" "F.Mask") (roundrect_rratio 0.1)
   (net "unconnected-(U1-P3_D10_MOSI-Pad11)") (thermal_bridge_angle 45))
  (pad "12" thru_hole circle (at 2.54 7.62 270) (size 1.524 1.524) (drill 0.889) (layers "*.Cu" "*.Mask") (remove_unused_layers no)
   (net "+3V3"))
  (pad "12" smd roundrect (at 2.54 8.455 270) (size 2.432 1.524) (layers "F.Cu" "F.Mask") (roundrect_rratio 0.1) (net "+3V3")
   (thermal_bridge_angle 45))
  (pad "13" thru_hole circle (at 5.08 7.62 270) (size 1.524 1.524) (drill 0.889) (layers "*.Cu" "*.Mask") (remove_unused_layers no)
   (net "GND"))
  (pad "13" smd roundrect (at 5.08 8.455 270) (size 2.432 1.524) (layers "F.Cu" "F.Mask") (roundrect_rratio 0.1) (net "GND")
   (thermal_bridge_angle 45))
  (pad "14" thru_hole circle (at 7.62 7.62 270) (size 1.524 1.524) (drill 0.889) (layers "*.Cu" "*.Mask") (remove_unused_layers no)
   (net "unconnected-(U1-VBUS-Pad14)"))
  (pad "14" smd roundrect (at 7.62 8.455 270) (size 2.432 1.524) (layers "F.Cu" "F.Mask") (roundrect_rratio 0.1)
   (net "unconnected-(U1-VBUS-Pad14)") (thermal_bridge_angle 45)))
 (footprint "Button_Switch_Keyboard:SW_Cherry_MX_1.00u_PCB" (layer "F.Cu") (at 128.115 121.395)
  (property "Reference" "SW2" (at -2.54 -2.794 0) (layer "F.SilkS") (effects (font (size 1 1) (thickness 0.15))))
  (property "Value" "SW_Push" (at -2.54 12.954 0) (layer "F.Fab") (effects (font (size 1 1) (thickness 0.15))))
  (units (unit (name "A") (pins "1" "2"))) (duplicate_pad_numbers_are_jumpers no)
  (fp_line (start -9.525 -1.905) (end 4.445 -1.905) (stroke (width 0.12) (type solid)) (layer "F.SilkS"))
  (fp_line (start -9.525 12.065) (end -9.525 -1.905) (stroke (width 0.12) (type solid)) (layer "F.SilkS"))
  (fp_line (start 4.445 -1.905) (end 4.445 12.065) (stroke (width 0.12) (type solid)) (layer "F.SilkS"))
  (fp_line (start 4.445 12.065) (end -9.525 12.065) (stroke (width 0.12) (type solid)) (layer "F.SilkS"))
  (pad "" np_thru_hole circle (at -7.62 5.08) (size 1.7 1.7) (drill 1.7) (layers "*.Cu" "*.Mask"))
  (pad "" np_thru_hole circle (at -2.54 5.08) (size 4 4) (drill 4) (layers "*.Cu" "*.Mask"))
  (pad "" np_thru_hole circle (at 2.54 5.08) (size 1.7 1.7) (drill 1.7) (layers "*.Cu" "*.Mask"))
  (pad "1" thru_hole circle (at 0 0) (size 2.2 2.2) (drill 1.5) (layers "*.Cu" "*.Mask") (remove_unused_layers no) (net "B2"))
  (pad "2" thru_hole circle (at -6.35 2.54) (size 2.2 2.2) (drill 1.5) (layers "*.Cu" "*.Mask") (remove_unused_layers no) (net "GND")))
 (gr_arc (start 95.001549 106.002976) (mid 95.587347 104.588795) (end 97.001549 104.002976) (stroke (width 0.05) (type default))
  (layer "Edge.Cuts"))
 (gr_line (start 95.001549 136) (end 95.001549 106.002976) (stroke (width 0.05) (type default)) (layer "Edge.Cuts"))
 (gr_line (start 97.001549 104.002976) (end 175.857722 104.002976) (stroke (width 0.05) (type default)) (layer "Edge.Cuts"))
 (gr_arc (start 97.001549 138) (mid 95.587335 137.414214) (end 95.001549 136) (stroke (width 0.05) (type default)) (layer "Edge.Cuts"))
 (gr_arc (start 175.857722 104.002976) (mid 177.271936 104.588762) (end 177.857722 106.002976) (stroke (width 0.05) (type default))
  (layer "Edge.Cuts"))
 (gr_line (start 175.857722 138) (end 97.001549 138) (stroke (width 0.05) (type default)) (layer "Edge.Cuts"))
 (gr_line (start 177.857722 106.002976) (end 177.857722 136) (stroke (width 0.05) (type default)) (layer "Edge.Cuts"))
 (gr_arc (start 177.857722 136) (mid 177.271937 137.414221) (end 175.857722 138) (stroke (width 0.05) (type default)) (layer "Edge.Cuts"))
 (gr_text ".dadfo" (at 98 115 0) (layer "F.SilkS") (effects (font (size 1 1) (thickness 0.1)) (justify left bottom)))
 (segment (start 162.8565 117.68575) (end 162.8565 119.515) (width 0.2) (layer "B.Cu") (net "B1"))
 (segment (start 161.89575 116.725) (end 162.8565 117.68575) (width 0.2) (layer "B.Cu") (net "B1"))
 (segment (start 109.065 121.395) (end 113.735 116.725) (width 0.2) (layer "B.Cu") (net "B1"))
 (segment (start 113.735 116.725) (end 161.89575 116.725) (width 0.2) (layer "B.Cu") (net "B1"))
 (segment (start 121.765 111.975) (end 121.765 123.935) (width 0.2) (layer "F.Cu") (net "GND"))
 (segment (start 124.305 109.435) (end 121.765 111.975) (width 0.2) (layer "F.Cu") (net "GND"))
 (segment (start 174.7 130.5315) (end 174.7 115.62) (width 0.2) (layer "F.Cu") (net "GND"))
 (segment (start 170.4765 134.755) (end 174.7 130.5315) (width 0.2) (layer "F.Cu") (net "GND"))
 (segment (start 174.7 115.62) (end 168.08 109) (width 0.2) (layer "F.Cu") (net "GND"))
 (segment (start 102.715 123.935) (end 121.765 123.935) (width 0.2) (layer "B.Cu") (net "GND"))
 (segment (start 105.255 121.395) (end 102.715 123.935) (width 0.2) (layer "B.Cu") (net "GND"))
 (segment (start 105.255 109.435) (end 105.255 121.395) (width 0.2) (layer "B.Cu") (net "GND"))
 (segment (start 139.29 113.5) (end 143.355 109.435) (width 0.2) (layer "B.Cu") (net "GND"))
 (segment (start 140.815 123.935) (end 163.044081 123.935) (width 0.2) (layer "B.Cu") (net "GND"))
 (segment (start 170.4765 134.755) (end 170.4765 131.367419) (width 0.2) (layer "B.Cu") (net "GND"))
 (segment (start 121.765 123.935) (end 140.815 123.935) (width 0.2) (layer "B.Cu") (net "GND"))
 (segment (start 170.4765 131.367419) (end 163.044081 123.935) (width 0.2) (layer "B.Cu") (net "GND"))
 (segment (start 128.37 113.5) (end 139.29 113.5) (width 0.2) (layer "B.Cu") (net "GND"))
 (segment (start 124.305 109.435) (end 128.37 113.5) (width 0.2) (layer "B.Cu") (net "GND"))
 (segment (start 107.795 109.435) (end 110.225 109.435) (width 0.2) (layer "F.Cu") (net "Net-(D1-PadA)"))
 (segment (start 110.225 109.435) (end 112.765 106.895) (width 0.2) (layer "F.Cu") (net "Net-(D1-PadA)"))
 (segment (start 170.4765 117.9765) (end 170.4765 119.515) (width 0.2) (layer "B.Cu") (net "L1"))
 (segment (start 167.5 115) (end 170.4765 117.9765) (width 0.2) (layer "B.Cu") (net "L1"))
 (segment (start 112.765 111.975) (end 115.79 115) (width 0.2) (layer "B.Cu") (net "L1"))
 (segment (start 115.79 115) (end 167.5 115) (width 0.2) (layer "B.Cu") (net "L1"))
 (segment (start 148.365 109.435) (end 150.865 106.935) (width 0.2) (layer "F.Cu") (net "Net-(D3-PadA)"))
 (segment (start 145.895 109.435) (end 148.365 109.435) (width 0.2) (layer "F.Cu") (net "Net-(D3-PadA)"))
 (segment (start 162.845 108.7875) (end 162.901214 108.7875) (width 0.2) (layer "F.Cu") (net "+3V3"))
 (segment (start 163 109) (end 169.225 115.225) (width 0.2) (layer "F.Cu") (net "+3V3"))
 (segment (start 169.225 133.4665) (end 167.9365 134.755) (width 0.2) (layer "F.Cu") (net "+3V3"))
 (segment (start 169.225 115.225) (end 169.225 133.4665) (width 0.2) (layer "F.Cu") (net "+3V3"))
 (segment (start 163 109) (end 163.375 109) (width 0.2) (layer "B.Cu") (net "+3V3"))
 (segment (start 165.54 109) (end 173.0165 116.4765) (width 0.2) (layer "B.Cu") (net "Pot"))
 (segment (start 173.0165 116.4765) (end 173.0165 119.515) (width 0.2) (layer "B.Cu") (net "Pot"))
 (segment (start 129.315 109.435) (end 131.815 106.935) (width 0.2) (layer "F.Cu") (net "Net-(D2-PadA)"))
 (segment (start 126.845 109.435) (end 129.315 109.435) (width 0.2) (layer "F.Cu") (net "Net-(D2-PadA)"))
 (segment (start 159.49913 110) (end 150 110) (width 0.2) (layer "F.Cu") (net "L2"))
 (segment (start 167.9365 119.515) (end 167.9365 118.43737) (width 0.2) (layer "F.Cu") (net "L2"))
 (segment (start 147.985 112.015) (end 131.815 112.015) (width 0.2) (layer "F.Cu") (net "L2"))
 (segment (start 150 110) (end 147.985 112.015) (width 0.2) (layer "F.Cu") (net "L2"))
 (segment (start 167.9365 118.43737) (end 159.49913 110) (width 0.2) (layer "F.Cu") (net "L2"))
 (segment (start 147.165 121.395) (end 155.8965 121.395) (width 0.2) (layer "B.Cu") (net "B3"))
 (segment (start 155.8965 121.395) (end 157.7765 119.515) (width 0.2) (layer "B.Cu") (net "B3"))
 (segment (start 165.3965 119.515) (end 165.3965 118.43737) (width 0.2) (layer "F.Cu") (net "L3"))
 (segment (start 165.3965 118.43737) (end 158.97413 112.015) (width 0.2) (layer "F.Cu") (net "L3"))
 (segment (start 158.97413 112.015) (end 150.865 112.015) (width 0.2) (layer "F.Cu") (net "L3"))
 (segment (start 165.3965 119.9035) (end 165.3965 119.515) (width 0.2) (layer "F.Cu") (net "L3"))
 (segment (start 158.5 116) (end 133.51 116) (width 0.2) (layer "F.Cu") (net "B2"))
 (segment (start 160.3165 117.8165) (end 158.5 116) (width 0.2) (layer "F.Cu") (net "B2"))
 (segment (start 160.3165 119.515) (end 160.3165 117.8165) (width 0.2) (layer "F.Cu") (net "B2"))
 (segment (start 160.3165 118.68) (end 160.3165 119.515) (width 0.2) (layer "F.Cu") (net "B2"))
 (segment (start 133.51 116) (end 128.115 121.395) (width 0.2) (layer "F.Cu") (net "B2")))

